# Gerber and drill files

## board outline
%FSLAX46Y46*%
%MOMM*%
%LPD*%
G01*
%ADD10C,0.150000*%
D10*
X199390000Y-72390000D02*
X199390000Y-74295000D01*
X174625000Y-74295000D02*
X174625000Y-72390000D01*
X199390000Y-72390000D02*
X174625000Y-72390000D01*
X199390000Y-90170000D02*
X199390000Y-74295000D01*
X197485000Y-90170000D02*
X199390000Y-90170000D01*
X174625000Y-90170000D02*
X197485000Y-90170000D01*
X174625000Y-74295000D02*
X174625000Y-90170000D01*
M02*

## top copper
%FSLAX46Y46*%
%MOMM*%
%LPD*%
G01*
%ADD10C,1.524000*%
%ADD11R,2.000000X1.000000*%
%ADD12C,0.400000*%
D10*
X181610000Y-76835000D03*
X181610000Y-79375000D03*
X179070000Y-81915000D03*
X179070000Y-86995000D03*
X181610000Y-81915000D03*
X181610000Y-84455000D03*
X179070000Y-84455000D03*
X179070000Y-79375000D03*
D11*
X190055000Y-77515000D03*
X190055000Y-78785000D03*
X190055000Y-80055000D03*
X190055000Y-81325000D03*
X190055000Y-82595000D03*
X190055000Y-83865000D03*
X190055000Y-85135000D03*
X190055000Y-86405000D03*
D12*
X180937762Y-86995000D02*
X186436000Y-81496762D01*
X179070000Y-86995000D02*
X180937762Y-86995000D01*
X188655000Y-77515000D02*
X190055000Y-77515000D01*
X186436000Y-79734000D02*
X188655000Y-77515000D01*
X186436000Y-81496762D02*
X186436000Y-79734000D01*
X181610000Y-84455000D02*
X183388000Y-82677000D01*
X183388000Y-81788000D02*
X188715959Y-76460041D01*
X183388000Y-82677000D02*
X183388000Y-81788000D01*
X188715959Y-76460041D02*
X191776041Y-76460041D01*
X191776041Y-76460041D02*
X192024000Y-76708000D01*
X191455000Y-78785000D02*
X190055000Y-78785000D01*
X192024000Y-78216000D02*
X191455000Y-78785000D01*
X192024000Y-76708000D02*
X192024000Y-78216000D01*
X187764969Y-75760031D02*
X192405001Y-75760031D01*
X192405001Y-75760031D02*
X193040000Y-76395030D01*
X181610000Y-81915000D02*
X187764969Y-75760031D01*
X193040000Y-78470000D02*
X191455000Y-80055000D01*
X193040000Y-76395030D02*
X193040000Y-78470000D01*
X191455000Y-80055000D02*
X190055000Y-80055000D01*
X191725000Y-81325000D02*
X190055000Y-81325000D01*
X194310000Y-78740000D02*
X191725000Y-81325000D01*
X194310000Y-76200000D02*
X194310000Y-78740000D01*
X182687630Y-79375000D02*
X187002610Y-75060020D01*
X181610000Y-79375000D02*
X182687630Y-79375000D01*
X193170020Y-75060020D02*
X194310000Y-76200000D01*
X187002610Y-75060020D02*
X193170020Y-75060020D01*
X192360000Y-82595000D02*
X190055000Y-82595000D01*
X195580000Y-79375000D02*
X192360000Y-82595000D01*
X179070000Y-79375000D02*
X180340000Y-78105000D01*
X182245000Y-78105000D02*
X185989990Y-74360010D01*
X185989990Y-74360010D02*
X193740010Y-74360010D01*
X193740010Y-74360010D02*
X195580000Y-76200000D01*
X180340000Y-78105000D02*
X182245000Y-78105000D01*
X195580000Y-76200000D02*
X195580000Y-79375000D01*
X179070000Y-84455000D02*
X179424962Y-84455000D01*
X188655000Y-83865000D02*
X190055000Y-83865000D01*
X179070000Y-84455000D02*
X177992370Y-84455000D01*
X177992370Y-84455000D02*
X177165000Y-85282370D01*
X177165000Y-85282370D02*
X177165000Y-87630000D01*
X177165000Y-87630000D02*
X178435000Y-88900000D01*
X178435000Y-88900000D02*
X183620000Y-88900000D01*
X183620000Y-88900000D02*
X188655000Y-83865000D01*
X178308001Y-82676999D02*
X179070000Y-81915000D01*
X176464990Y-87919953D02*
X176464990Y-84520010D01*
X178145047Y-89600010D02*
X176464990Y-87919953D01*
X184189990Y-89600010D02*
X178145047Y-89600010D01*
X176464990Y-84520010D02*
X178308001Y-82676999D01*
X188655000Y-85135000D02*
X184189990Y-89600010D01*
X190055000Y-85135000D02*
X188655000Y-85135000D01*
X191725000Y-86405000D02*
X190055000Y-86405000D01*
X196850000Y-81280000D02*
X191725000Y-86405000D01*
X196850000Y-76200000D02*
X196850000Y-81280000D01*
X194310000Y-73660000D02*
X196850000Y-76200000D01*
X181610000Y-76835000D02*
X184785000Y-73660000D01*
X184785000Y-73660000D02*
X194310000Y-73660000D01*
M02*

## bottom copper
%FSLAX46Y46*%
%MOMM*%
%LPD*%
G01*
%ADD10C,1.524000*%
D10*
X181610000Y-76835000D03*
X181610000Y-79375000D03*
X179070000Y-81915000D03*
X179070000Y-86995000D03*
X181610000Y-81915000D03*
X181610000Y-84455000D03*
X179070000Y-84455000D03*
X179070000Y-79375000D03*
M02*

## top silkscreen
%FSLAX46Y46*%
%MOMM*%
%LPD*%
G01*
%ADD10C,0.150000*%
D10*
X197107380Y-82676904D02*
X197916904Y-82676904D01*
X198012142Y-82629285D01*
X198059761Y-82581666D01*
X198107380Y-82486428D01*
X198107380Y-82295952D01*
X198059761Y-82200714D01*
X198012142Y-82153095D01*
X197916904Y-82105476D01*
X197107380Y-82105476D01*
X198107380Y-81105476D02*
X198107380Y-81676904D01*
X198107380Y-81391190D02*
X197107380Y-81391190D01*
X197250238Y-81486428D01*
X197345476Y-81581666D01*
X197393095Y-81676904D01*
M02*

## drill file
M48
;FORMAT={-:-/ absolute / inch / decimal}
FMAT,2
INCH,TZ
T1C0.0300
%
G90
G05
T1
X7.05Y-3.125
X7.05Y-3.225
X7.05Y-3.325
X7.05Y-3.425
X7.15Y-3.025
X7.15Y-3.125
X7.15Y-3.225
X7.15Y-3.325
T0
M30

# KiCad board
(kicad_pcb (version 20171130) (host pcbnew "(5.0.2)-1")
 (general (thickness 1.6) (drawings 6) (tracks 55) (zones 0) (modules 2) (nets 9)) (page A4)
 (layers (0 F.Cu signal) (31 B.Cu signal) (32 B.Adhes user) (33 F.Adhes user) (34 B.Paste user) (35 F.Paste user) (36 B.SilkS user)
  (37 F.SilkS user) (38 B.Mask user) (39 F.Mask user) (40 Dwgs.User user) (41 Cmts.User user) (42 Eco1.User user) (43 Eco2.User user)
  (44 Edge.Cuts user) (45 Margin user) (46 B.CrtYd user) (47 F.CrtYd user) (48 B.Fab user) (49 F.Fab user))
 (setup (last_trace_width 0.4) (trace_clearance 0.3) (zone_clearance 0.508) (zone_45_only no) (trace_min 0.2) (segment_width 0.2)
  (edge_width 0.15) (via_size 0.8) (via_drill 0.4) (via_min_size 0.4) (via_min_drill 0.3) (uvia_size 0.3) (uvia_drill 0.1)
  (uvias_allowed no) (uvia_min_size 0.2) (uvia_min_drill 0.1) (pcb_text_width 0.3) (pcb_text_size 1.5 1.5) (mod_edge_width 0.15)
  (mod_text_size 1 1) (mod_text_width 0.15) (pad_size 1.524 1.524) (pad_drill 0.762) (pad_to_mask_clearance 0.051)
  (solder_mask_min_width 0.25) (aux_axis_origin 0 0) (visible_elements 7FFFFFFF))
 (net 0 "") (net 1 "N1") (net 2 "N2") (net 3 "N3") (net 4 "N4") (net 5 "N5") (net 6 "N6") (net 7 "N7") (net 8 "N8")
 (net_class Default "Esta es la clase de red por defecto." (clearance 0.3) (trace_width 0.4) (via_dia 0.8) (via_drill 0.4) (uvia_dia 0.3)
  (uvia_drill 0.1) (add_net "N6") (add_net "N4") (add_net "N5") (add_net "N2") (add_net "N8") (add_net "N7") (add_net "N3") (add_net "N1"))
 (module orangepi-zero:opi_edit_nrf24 (layer B.Cu) (at 180.34 73.025 180)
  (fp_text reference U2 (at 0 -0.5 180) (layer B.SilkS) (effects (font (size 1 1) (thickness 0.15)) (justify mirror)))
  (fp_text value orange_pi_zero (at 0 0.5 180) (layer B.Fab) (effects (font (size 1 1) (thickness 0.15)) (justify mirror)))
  (pad 126 thru_hole circle (at -1.27 -3.81 180) (size 1.524 1.524) (drill 0.762) (layers *.Cu *.Mask B.SilkS) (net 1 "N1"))
  (pad 124 thru_hole circle (at -1.27 -6.35 180) (size 1.524 1.524) (drill 0.762) (layers *.Cu *.Mask B.SilkS) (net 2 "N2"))
  (pad 121 thru_hole circle (at 1.27 -8.89 180) (size 1.524 1.524) (drill 0.762) (layers *.Cu *.Mask B.SilkS) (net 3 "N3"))
  (pad 117 thru_hole circle (at 1.27 -13.97 180) (size 1.524 1.524) (drill 0.762) (layers *.Cu *.Mask B.SilkS) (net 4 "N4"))
  (pad 122 thru_hole circle (at -1.27 -8.89 180) (size 1.524 1.524) (drill 0.762) (layers *.Cu *.Mask B.SilkS) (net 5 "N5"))
  (pad 120 thru_hole circle (at -1.27 -11.43 180) (size 1.524 1.524) (drill 0.762) (layers *.Cu *.Mask B.SilkS) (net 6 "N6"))
  (pad 119 thru_hole circle (at 1.27 -11.43 180) (size 1.524 1.524) (drill 0.762) (layers *.Cu *.Mask B.SilkS) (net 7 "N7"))
  (pad 123 thru_hole circle (at 1.27 -6.35 180) (size 1.524 1.524) (drill 0.762) (layers *.Cu *.Mask B.SilkS) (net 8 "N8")))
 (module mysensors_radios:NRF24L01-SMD (layer F.Cu) (at 198.755 81.915 270)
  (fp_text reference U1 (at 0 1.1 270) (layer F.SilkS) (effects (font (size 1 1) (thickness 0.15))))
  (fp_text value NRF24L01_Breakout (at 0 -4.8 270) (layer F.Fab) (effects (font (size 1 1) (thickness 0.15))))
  (pad 2 smd rect (at -4.4 8.7 270) (size 1 2) (layers F.Cu F.Paste F.Mask) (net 4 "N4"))
  (pad 1 smd rect (at -3.13 8.7 270) (size 1 2) (layers F.Cu F.Paste F.Mask) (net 6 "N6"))
  (pad 3 smd rect (at -1.86 8.7 270) (size 1 2) (layers F.Cu F.Paste F.Mask) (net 5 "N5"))
  (pad 4 smd rect (at -0.59 8.7 270) (size 1 2) (layers F.Cu F.Paste F.Mask) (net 2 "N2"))
  (pad 5 smd rect (at 0.68 8.7 270) (size 1 2) (layers F.Cu F.Paste F.Mask) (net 8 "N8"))
  (pad 6 smd rect (at 1.95 8.7 270) (size 1 2) (layers F.Cu F.Paste F.Mask) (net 7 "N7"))
  (pad 7 smd rect (at 3.22 8.7 270) (size 1 2) (layers F.Cu F.Paste F.Mask) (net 3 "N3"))
  (pad 8 smd rect (at 4.49 8.7 270) (size 1 2) (layers F.Cu F.Paste F.Mask) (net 1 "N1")))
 (gr_line (start 174.625 74.295) (end 174.625 72.39) (layer Edge.Cuts) (width 0.15))
 (gr_line (start 199.39 72.39) (end 174.625 72.39) (layer Edge.Cuts) (width 0.15))
 (gr_line (start 199.39 90.17) (end 199.39 72.39) (layer Edge.Cuts) (width 0.15))
 (gr_line (start 197.485 90.17) (end 199.39 90.17) (layer Edge.Cuts) (width 0.15))
 (gr_line (start 174.625 90.17) (end 197.485 90.17) (layer Edge.Cuts) (width 0.15))
 (gr_line (start 174.625 74.295) (end 174.625 90.17) (layer Edge.Cuts) (width 0.15))
 (segment (start 180.937762 86.995) (end 186.436 81.496762) (width 0.4) (layer F.Cu) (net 4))
 (segment (start 179.07 86.995) (end 180.937762 86.995) (width 0.4) (layer F.Cu) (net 4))
 (segment (start 188.655 77.515) (end 190.055 77.515) (width 0.4) (layer F.Cu) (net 4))
 (segment (start 186.436 79.734) (end 188.655 77.515) (width 0.4) (layer F.Cu) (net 4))
 (segment (start 186.436 81.496762) (end 186.436 79.734) (width 0.4) (layer F.Cu) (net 4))
 (segment (start 181.61 84.455) (end 183.388 82.677) (width 0.4) (layer F.Cu) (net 6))
 (segment (start 183.388 81.788) (end 188.715959 76.460041) (width 0.4) (layer F.Cu) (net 6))
 (segment (start 183.388 82.677) (end 183.388 81.788) (width 0.4) (layer F.Cu) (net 6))
 (segment (start 188.715959 76.460041) (end 191.776041 76.460041) (width 0.4) (layer F.Cu) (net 6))
 (segment (start 191.776041 76.460041) (end 192.024 76.708) (width 0.4) (layer F.Cu) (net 6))
 (segment (start 191.455 78.785) (end 190.055 78.785) (width 0.4) (layer F.Cu) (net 6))
 (segment (start 192.024 78.216) (end 191.455 78.785) (width 0.4) (layer F.Cu) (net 6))
 (segment (start 192.024 76.708) (end 192.024 78.216) (width 0.4) (layer F.Cu) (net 6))
 (segment (start 187.764969 75.760031) (end 192.405001 75.760031) (width 0.4) (layer F.Cu) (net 5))
 (segment (start 192.405001 75.760031) (end 193.04 76.39503) (width 0.4) (layer F.Cu) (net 5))
 (segment (start 181.61 81.915) (end 187.764969 75.760031) (width 0.4) (layer F.Cu) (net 5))
 (segment (start 193.04 78.47) (end 191.455 80.055) (width 0.4) (layer F.Cu) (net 5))
 (segment (start 193.04 76.39503) (end 193.04 78.47) (width 0.4) (layer F.Cu) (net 5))
 (segment (start 191.455 80.055) (end 190.055 80.055) (width 0.4) (layer F.Cu) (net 5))
 (segment (start 191.725 81.325) (end 190.055 81.325) (width 0.4) (layer F.Cu) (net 2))
 (segment (start 194.31 78.74) (end 191.725 81.325) (width 0.4) (layer F.Cu) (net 2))
 (segment (start 194.31 76.2) (end 194.31 78.74) (width 0.4) (layer F.Cu) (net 2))
 (segment (start 182.68763 79.375) (end 187.00261 75.06002) (width 0.4) (layer F.Cu) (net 2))
 (segment (start 181.61 79.375) (end 182.68763 79.375) (width 0.4) (layer F.Cu) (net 2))
 (segment (start 193.17002 75.06002) (end 194.31 76.2) (width 0.4) (layer F.Cu) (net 2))
 (segment (start 187.00261 75.06002) (end 193.17002 75.06002) (width 0.4) (layer F.Cu) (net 2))
 (segment (start 192.36 82.595) (end 190.055 82.595) (width 0.4) (layer F.Cu) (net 8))
 (segment (start 195.58 79.375) (end 192.36 82.595) (width 0.4) (layer F.Cu) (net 8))
 (segment (start 179.07 79.375) (end 180.34 78.105) (width 0.4) (layer F.Cu) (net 8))
 (segment (start 182.245 78.105) (end 185.98999 74.36001) (width 0.4) (layer F.Cu) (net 8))
 (segment (start 185.98999 74.36001) (end 193.74001 74.36001) (width 0.4) (layer F.Cu) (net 8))
 (segment (start 193.74001 74.36001) (end 195.58 76.2) (width 0.4) (layer F.Cu) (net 8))
 (segment (start 180.34 78.105) (end 182.245 78.105) (width 0.4) (layer F.Cu) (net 8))
 (segment (start 195.58 76.2) (end 195.58 79.375) (width 0.4) (layer F.Cu) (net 8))
 (segment (start 179.07 84.455) (end 179.424962 84.455) (width 0.4) (layer F.Cu) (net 7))
 (segment (start 188.655 83.865) (end 190.055 83.865) (width 0.4) (layer F.Cu) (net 7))
 (segment (start 179.07 84.455) (end 177.99237 84.455) (width 0.4) (layer F.Cu) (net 7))
 (segment (start 177.99237 84.455) (end 177.165 85.28237) (width 0.4) (layer F.Cu) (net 7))
 (segment (start 177.165 85.28237) (end 177.165 87.63) (width 0.4) (layer F.Cu) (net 7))
 (segment (start 177.165 87.63) (end 178.435 88.9) (width 0.4) (layer F.Cu) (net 7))
 (segment (start 178.435 88.9) (end 183.62 88.9) (width 0.4) (layer F.Cu) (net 7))
 (segment (start 183.62 88.9) (end 188.655 83.865) (width 0.4) (layer F.Cu) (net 7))
 (segment (start 178.308001 82.676999) (end 179.07 81.915) (width 0.4) (layer F.Cu) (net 3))
 (segment (start 176.46499 87.919953) (end 176.46499 84.52001) (width 0.4) (layer F.Cu) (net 3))
 (segment (start 178.145047 89.60001) (end 176.46499 87.919953) (width 0.4) (layer F.Cu) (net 3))
 (segment (start 184.18999 89.60001) (end 178.145047 89.60001) (width 0.4) (layer F.Cu) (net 3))
 (segment (start 176.46499 84.52001) (end 178.308001 82.676999) (width 0.4) (layer F.Cu) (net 3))
 (segment (start 188.655 85.135) (end 184.18999 89.60001) (width 0.4) (layer F.Cu) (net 3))
 (segment (start 190.055 85.135) (end 188.655 85.135) (width 0.4) (layer F.Cu) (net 3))
 (segment (start 191.725 86.405) (end 190.055 86.405) (width 0.4) (layer F.Cu) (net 1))
 (segment (start 196.85 81.28) (end 191.725 86.405) (width 0.4) (layer F.Cu) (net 1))
 (segment (start 196.85 76.2) (end 196.85 81.28) (width 0.4) (layer F.Cu) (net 1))
 (segment (start 194.31 73.66) (end 196.85 76.2) (width 0.4) (layer F.Cu) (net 1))
 (segment (start 181.61 76.835) (end 184.785 73.66) (width 0.4) (layer F.Cu) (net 1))
 (segment (start 184.785 73.66) (end 194.31 73.66) (width 0.4) (layer F.Cu) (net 1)))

